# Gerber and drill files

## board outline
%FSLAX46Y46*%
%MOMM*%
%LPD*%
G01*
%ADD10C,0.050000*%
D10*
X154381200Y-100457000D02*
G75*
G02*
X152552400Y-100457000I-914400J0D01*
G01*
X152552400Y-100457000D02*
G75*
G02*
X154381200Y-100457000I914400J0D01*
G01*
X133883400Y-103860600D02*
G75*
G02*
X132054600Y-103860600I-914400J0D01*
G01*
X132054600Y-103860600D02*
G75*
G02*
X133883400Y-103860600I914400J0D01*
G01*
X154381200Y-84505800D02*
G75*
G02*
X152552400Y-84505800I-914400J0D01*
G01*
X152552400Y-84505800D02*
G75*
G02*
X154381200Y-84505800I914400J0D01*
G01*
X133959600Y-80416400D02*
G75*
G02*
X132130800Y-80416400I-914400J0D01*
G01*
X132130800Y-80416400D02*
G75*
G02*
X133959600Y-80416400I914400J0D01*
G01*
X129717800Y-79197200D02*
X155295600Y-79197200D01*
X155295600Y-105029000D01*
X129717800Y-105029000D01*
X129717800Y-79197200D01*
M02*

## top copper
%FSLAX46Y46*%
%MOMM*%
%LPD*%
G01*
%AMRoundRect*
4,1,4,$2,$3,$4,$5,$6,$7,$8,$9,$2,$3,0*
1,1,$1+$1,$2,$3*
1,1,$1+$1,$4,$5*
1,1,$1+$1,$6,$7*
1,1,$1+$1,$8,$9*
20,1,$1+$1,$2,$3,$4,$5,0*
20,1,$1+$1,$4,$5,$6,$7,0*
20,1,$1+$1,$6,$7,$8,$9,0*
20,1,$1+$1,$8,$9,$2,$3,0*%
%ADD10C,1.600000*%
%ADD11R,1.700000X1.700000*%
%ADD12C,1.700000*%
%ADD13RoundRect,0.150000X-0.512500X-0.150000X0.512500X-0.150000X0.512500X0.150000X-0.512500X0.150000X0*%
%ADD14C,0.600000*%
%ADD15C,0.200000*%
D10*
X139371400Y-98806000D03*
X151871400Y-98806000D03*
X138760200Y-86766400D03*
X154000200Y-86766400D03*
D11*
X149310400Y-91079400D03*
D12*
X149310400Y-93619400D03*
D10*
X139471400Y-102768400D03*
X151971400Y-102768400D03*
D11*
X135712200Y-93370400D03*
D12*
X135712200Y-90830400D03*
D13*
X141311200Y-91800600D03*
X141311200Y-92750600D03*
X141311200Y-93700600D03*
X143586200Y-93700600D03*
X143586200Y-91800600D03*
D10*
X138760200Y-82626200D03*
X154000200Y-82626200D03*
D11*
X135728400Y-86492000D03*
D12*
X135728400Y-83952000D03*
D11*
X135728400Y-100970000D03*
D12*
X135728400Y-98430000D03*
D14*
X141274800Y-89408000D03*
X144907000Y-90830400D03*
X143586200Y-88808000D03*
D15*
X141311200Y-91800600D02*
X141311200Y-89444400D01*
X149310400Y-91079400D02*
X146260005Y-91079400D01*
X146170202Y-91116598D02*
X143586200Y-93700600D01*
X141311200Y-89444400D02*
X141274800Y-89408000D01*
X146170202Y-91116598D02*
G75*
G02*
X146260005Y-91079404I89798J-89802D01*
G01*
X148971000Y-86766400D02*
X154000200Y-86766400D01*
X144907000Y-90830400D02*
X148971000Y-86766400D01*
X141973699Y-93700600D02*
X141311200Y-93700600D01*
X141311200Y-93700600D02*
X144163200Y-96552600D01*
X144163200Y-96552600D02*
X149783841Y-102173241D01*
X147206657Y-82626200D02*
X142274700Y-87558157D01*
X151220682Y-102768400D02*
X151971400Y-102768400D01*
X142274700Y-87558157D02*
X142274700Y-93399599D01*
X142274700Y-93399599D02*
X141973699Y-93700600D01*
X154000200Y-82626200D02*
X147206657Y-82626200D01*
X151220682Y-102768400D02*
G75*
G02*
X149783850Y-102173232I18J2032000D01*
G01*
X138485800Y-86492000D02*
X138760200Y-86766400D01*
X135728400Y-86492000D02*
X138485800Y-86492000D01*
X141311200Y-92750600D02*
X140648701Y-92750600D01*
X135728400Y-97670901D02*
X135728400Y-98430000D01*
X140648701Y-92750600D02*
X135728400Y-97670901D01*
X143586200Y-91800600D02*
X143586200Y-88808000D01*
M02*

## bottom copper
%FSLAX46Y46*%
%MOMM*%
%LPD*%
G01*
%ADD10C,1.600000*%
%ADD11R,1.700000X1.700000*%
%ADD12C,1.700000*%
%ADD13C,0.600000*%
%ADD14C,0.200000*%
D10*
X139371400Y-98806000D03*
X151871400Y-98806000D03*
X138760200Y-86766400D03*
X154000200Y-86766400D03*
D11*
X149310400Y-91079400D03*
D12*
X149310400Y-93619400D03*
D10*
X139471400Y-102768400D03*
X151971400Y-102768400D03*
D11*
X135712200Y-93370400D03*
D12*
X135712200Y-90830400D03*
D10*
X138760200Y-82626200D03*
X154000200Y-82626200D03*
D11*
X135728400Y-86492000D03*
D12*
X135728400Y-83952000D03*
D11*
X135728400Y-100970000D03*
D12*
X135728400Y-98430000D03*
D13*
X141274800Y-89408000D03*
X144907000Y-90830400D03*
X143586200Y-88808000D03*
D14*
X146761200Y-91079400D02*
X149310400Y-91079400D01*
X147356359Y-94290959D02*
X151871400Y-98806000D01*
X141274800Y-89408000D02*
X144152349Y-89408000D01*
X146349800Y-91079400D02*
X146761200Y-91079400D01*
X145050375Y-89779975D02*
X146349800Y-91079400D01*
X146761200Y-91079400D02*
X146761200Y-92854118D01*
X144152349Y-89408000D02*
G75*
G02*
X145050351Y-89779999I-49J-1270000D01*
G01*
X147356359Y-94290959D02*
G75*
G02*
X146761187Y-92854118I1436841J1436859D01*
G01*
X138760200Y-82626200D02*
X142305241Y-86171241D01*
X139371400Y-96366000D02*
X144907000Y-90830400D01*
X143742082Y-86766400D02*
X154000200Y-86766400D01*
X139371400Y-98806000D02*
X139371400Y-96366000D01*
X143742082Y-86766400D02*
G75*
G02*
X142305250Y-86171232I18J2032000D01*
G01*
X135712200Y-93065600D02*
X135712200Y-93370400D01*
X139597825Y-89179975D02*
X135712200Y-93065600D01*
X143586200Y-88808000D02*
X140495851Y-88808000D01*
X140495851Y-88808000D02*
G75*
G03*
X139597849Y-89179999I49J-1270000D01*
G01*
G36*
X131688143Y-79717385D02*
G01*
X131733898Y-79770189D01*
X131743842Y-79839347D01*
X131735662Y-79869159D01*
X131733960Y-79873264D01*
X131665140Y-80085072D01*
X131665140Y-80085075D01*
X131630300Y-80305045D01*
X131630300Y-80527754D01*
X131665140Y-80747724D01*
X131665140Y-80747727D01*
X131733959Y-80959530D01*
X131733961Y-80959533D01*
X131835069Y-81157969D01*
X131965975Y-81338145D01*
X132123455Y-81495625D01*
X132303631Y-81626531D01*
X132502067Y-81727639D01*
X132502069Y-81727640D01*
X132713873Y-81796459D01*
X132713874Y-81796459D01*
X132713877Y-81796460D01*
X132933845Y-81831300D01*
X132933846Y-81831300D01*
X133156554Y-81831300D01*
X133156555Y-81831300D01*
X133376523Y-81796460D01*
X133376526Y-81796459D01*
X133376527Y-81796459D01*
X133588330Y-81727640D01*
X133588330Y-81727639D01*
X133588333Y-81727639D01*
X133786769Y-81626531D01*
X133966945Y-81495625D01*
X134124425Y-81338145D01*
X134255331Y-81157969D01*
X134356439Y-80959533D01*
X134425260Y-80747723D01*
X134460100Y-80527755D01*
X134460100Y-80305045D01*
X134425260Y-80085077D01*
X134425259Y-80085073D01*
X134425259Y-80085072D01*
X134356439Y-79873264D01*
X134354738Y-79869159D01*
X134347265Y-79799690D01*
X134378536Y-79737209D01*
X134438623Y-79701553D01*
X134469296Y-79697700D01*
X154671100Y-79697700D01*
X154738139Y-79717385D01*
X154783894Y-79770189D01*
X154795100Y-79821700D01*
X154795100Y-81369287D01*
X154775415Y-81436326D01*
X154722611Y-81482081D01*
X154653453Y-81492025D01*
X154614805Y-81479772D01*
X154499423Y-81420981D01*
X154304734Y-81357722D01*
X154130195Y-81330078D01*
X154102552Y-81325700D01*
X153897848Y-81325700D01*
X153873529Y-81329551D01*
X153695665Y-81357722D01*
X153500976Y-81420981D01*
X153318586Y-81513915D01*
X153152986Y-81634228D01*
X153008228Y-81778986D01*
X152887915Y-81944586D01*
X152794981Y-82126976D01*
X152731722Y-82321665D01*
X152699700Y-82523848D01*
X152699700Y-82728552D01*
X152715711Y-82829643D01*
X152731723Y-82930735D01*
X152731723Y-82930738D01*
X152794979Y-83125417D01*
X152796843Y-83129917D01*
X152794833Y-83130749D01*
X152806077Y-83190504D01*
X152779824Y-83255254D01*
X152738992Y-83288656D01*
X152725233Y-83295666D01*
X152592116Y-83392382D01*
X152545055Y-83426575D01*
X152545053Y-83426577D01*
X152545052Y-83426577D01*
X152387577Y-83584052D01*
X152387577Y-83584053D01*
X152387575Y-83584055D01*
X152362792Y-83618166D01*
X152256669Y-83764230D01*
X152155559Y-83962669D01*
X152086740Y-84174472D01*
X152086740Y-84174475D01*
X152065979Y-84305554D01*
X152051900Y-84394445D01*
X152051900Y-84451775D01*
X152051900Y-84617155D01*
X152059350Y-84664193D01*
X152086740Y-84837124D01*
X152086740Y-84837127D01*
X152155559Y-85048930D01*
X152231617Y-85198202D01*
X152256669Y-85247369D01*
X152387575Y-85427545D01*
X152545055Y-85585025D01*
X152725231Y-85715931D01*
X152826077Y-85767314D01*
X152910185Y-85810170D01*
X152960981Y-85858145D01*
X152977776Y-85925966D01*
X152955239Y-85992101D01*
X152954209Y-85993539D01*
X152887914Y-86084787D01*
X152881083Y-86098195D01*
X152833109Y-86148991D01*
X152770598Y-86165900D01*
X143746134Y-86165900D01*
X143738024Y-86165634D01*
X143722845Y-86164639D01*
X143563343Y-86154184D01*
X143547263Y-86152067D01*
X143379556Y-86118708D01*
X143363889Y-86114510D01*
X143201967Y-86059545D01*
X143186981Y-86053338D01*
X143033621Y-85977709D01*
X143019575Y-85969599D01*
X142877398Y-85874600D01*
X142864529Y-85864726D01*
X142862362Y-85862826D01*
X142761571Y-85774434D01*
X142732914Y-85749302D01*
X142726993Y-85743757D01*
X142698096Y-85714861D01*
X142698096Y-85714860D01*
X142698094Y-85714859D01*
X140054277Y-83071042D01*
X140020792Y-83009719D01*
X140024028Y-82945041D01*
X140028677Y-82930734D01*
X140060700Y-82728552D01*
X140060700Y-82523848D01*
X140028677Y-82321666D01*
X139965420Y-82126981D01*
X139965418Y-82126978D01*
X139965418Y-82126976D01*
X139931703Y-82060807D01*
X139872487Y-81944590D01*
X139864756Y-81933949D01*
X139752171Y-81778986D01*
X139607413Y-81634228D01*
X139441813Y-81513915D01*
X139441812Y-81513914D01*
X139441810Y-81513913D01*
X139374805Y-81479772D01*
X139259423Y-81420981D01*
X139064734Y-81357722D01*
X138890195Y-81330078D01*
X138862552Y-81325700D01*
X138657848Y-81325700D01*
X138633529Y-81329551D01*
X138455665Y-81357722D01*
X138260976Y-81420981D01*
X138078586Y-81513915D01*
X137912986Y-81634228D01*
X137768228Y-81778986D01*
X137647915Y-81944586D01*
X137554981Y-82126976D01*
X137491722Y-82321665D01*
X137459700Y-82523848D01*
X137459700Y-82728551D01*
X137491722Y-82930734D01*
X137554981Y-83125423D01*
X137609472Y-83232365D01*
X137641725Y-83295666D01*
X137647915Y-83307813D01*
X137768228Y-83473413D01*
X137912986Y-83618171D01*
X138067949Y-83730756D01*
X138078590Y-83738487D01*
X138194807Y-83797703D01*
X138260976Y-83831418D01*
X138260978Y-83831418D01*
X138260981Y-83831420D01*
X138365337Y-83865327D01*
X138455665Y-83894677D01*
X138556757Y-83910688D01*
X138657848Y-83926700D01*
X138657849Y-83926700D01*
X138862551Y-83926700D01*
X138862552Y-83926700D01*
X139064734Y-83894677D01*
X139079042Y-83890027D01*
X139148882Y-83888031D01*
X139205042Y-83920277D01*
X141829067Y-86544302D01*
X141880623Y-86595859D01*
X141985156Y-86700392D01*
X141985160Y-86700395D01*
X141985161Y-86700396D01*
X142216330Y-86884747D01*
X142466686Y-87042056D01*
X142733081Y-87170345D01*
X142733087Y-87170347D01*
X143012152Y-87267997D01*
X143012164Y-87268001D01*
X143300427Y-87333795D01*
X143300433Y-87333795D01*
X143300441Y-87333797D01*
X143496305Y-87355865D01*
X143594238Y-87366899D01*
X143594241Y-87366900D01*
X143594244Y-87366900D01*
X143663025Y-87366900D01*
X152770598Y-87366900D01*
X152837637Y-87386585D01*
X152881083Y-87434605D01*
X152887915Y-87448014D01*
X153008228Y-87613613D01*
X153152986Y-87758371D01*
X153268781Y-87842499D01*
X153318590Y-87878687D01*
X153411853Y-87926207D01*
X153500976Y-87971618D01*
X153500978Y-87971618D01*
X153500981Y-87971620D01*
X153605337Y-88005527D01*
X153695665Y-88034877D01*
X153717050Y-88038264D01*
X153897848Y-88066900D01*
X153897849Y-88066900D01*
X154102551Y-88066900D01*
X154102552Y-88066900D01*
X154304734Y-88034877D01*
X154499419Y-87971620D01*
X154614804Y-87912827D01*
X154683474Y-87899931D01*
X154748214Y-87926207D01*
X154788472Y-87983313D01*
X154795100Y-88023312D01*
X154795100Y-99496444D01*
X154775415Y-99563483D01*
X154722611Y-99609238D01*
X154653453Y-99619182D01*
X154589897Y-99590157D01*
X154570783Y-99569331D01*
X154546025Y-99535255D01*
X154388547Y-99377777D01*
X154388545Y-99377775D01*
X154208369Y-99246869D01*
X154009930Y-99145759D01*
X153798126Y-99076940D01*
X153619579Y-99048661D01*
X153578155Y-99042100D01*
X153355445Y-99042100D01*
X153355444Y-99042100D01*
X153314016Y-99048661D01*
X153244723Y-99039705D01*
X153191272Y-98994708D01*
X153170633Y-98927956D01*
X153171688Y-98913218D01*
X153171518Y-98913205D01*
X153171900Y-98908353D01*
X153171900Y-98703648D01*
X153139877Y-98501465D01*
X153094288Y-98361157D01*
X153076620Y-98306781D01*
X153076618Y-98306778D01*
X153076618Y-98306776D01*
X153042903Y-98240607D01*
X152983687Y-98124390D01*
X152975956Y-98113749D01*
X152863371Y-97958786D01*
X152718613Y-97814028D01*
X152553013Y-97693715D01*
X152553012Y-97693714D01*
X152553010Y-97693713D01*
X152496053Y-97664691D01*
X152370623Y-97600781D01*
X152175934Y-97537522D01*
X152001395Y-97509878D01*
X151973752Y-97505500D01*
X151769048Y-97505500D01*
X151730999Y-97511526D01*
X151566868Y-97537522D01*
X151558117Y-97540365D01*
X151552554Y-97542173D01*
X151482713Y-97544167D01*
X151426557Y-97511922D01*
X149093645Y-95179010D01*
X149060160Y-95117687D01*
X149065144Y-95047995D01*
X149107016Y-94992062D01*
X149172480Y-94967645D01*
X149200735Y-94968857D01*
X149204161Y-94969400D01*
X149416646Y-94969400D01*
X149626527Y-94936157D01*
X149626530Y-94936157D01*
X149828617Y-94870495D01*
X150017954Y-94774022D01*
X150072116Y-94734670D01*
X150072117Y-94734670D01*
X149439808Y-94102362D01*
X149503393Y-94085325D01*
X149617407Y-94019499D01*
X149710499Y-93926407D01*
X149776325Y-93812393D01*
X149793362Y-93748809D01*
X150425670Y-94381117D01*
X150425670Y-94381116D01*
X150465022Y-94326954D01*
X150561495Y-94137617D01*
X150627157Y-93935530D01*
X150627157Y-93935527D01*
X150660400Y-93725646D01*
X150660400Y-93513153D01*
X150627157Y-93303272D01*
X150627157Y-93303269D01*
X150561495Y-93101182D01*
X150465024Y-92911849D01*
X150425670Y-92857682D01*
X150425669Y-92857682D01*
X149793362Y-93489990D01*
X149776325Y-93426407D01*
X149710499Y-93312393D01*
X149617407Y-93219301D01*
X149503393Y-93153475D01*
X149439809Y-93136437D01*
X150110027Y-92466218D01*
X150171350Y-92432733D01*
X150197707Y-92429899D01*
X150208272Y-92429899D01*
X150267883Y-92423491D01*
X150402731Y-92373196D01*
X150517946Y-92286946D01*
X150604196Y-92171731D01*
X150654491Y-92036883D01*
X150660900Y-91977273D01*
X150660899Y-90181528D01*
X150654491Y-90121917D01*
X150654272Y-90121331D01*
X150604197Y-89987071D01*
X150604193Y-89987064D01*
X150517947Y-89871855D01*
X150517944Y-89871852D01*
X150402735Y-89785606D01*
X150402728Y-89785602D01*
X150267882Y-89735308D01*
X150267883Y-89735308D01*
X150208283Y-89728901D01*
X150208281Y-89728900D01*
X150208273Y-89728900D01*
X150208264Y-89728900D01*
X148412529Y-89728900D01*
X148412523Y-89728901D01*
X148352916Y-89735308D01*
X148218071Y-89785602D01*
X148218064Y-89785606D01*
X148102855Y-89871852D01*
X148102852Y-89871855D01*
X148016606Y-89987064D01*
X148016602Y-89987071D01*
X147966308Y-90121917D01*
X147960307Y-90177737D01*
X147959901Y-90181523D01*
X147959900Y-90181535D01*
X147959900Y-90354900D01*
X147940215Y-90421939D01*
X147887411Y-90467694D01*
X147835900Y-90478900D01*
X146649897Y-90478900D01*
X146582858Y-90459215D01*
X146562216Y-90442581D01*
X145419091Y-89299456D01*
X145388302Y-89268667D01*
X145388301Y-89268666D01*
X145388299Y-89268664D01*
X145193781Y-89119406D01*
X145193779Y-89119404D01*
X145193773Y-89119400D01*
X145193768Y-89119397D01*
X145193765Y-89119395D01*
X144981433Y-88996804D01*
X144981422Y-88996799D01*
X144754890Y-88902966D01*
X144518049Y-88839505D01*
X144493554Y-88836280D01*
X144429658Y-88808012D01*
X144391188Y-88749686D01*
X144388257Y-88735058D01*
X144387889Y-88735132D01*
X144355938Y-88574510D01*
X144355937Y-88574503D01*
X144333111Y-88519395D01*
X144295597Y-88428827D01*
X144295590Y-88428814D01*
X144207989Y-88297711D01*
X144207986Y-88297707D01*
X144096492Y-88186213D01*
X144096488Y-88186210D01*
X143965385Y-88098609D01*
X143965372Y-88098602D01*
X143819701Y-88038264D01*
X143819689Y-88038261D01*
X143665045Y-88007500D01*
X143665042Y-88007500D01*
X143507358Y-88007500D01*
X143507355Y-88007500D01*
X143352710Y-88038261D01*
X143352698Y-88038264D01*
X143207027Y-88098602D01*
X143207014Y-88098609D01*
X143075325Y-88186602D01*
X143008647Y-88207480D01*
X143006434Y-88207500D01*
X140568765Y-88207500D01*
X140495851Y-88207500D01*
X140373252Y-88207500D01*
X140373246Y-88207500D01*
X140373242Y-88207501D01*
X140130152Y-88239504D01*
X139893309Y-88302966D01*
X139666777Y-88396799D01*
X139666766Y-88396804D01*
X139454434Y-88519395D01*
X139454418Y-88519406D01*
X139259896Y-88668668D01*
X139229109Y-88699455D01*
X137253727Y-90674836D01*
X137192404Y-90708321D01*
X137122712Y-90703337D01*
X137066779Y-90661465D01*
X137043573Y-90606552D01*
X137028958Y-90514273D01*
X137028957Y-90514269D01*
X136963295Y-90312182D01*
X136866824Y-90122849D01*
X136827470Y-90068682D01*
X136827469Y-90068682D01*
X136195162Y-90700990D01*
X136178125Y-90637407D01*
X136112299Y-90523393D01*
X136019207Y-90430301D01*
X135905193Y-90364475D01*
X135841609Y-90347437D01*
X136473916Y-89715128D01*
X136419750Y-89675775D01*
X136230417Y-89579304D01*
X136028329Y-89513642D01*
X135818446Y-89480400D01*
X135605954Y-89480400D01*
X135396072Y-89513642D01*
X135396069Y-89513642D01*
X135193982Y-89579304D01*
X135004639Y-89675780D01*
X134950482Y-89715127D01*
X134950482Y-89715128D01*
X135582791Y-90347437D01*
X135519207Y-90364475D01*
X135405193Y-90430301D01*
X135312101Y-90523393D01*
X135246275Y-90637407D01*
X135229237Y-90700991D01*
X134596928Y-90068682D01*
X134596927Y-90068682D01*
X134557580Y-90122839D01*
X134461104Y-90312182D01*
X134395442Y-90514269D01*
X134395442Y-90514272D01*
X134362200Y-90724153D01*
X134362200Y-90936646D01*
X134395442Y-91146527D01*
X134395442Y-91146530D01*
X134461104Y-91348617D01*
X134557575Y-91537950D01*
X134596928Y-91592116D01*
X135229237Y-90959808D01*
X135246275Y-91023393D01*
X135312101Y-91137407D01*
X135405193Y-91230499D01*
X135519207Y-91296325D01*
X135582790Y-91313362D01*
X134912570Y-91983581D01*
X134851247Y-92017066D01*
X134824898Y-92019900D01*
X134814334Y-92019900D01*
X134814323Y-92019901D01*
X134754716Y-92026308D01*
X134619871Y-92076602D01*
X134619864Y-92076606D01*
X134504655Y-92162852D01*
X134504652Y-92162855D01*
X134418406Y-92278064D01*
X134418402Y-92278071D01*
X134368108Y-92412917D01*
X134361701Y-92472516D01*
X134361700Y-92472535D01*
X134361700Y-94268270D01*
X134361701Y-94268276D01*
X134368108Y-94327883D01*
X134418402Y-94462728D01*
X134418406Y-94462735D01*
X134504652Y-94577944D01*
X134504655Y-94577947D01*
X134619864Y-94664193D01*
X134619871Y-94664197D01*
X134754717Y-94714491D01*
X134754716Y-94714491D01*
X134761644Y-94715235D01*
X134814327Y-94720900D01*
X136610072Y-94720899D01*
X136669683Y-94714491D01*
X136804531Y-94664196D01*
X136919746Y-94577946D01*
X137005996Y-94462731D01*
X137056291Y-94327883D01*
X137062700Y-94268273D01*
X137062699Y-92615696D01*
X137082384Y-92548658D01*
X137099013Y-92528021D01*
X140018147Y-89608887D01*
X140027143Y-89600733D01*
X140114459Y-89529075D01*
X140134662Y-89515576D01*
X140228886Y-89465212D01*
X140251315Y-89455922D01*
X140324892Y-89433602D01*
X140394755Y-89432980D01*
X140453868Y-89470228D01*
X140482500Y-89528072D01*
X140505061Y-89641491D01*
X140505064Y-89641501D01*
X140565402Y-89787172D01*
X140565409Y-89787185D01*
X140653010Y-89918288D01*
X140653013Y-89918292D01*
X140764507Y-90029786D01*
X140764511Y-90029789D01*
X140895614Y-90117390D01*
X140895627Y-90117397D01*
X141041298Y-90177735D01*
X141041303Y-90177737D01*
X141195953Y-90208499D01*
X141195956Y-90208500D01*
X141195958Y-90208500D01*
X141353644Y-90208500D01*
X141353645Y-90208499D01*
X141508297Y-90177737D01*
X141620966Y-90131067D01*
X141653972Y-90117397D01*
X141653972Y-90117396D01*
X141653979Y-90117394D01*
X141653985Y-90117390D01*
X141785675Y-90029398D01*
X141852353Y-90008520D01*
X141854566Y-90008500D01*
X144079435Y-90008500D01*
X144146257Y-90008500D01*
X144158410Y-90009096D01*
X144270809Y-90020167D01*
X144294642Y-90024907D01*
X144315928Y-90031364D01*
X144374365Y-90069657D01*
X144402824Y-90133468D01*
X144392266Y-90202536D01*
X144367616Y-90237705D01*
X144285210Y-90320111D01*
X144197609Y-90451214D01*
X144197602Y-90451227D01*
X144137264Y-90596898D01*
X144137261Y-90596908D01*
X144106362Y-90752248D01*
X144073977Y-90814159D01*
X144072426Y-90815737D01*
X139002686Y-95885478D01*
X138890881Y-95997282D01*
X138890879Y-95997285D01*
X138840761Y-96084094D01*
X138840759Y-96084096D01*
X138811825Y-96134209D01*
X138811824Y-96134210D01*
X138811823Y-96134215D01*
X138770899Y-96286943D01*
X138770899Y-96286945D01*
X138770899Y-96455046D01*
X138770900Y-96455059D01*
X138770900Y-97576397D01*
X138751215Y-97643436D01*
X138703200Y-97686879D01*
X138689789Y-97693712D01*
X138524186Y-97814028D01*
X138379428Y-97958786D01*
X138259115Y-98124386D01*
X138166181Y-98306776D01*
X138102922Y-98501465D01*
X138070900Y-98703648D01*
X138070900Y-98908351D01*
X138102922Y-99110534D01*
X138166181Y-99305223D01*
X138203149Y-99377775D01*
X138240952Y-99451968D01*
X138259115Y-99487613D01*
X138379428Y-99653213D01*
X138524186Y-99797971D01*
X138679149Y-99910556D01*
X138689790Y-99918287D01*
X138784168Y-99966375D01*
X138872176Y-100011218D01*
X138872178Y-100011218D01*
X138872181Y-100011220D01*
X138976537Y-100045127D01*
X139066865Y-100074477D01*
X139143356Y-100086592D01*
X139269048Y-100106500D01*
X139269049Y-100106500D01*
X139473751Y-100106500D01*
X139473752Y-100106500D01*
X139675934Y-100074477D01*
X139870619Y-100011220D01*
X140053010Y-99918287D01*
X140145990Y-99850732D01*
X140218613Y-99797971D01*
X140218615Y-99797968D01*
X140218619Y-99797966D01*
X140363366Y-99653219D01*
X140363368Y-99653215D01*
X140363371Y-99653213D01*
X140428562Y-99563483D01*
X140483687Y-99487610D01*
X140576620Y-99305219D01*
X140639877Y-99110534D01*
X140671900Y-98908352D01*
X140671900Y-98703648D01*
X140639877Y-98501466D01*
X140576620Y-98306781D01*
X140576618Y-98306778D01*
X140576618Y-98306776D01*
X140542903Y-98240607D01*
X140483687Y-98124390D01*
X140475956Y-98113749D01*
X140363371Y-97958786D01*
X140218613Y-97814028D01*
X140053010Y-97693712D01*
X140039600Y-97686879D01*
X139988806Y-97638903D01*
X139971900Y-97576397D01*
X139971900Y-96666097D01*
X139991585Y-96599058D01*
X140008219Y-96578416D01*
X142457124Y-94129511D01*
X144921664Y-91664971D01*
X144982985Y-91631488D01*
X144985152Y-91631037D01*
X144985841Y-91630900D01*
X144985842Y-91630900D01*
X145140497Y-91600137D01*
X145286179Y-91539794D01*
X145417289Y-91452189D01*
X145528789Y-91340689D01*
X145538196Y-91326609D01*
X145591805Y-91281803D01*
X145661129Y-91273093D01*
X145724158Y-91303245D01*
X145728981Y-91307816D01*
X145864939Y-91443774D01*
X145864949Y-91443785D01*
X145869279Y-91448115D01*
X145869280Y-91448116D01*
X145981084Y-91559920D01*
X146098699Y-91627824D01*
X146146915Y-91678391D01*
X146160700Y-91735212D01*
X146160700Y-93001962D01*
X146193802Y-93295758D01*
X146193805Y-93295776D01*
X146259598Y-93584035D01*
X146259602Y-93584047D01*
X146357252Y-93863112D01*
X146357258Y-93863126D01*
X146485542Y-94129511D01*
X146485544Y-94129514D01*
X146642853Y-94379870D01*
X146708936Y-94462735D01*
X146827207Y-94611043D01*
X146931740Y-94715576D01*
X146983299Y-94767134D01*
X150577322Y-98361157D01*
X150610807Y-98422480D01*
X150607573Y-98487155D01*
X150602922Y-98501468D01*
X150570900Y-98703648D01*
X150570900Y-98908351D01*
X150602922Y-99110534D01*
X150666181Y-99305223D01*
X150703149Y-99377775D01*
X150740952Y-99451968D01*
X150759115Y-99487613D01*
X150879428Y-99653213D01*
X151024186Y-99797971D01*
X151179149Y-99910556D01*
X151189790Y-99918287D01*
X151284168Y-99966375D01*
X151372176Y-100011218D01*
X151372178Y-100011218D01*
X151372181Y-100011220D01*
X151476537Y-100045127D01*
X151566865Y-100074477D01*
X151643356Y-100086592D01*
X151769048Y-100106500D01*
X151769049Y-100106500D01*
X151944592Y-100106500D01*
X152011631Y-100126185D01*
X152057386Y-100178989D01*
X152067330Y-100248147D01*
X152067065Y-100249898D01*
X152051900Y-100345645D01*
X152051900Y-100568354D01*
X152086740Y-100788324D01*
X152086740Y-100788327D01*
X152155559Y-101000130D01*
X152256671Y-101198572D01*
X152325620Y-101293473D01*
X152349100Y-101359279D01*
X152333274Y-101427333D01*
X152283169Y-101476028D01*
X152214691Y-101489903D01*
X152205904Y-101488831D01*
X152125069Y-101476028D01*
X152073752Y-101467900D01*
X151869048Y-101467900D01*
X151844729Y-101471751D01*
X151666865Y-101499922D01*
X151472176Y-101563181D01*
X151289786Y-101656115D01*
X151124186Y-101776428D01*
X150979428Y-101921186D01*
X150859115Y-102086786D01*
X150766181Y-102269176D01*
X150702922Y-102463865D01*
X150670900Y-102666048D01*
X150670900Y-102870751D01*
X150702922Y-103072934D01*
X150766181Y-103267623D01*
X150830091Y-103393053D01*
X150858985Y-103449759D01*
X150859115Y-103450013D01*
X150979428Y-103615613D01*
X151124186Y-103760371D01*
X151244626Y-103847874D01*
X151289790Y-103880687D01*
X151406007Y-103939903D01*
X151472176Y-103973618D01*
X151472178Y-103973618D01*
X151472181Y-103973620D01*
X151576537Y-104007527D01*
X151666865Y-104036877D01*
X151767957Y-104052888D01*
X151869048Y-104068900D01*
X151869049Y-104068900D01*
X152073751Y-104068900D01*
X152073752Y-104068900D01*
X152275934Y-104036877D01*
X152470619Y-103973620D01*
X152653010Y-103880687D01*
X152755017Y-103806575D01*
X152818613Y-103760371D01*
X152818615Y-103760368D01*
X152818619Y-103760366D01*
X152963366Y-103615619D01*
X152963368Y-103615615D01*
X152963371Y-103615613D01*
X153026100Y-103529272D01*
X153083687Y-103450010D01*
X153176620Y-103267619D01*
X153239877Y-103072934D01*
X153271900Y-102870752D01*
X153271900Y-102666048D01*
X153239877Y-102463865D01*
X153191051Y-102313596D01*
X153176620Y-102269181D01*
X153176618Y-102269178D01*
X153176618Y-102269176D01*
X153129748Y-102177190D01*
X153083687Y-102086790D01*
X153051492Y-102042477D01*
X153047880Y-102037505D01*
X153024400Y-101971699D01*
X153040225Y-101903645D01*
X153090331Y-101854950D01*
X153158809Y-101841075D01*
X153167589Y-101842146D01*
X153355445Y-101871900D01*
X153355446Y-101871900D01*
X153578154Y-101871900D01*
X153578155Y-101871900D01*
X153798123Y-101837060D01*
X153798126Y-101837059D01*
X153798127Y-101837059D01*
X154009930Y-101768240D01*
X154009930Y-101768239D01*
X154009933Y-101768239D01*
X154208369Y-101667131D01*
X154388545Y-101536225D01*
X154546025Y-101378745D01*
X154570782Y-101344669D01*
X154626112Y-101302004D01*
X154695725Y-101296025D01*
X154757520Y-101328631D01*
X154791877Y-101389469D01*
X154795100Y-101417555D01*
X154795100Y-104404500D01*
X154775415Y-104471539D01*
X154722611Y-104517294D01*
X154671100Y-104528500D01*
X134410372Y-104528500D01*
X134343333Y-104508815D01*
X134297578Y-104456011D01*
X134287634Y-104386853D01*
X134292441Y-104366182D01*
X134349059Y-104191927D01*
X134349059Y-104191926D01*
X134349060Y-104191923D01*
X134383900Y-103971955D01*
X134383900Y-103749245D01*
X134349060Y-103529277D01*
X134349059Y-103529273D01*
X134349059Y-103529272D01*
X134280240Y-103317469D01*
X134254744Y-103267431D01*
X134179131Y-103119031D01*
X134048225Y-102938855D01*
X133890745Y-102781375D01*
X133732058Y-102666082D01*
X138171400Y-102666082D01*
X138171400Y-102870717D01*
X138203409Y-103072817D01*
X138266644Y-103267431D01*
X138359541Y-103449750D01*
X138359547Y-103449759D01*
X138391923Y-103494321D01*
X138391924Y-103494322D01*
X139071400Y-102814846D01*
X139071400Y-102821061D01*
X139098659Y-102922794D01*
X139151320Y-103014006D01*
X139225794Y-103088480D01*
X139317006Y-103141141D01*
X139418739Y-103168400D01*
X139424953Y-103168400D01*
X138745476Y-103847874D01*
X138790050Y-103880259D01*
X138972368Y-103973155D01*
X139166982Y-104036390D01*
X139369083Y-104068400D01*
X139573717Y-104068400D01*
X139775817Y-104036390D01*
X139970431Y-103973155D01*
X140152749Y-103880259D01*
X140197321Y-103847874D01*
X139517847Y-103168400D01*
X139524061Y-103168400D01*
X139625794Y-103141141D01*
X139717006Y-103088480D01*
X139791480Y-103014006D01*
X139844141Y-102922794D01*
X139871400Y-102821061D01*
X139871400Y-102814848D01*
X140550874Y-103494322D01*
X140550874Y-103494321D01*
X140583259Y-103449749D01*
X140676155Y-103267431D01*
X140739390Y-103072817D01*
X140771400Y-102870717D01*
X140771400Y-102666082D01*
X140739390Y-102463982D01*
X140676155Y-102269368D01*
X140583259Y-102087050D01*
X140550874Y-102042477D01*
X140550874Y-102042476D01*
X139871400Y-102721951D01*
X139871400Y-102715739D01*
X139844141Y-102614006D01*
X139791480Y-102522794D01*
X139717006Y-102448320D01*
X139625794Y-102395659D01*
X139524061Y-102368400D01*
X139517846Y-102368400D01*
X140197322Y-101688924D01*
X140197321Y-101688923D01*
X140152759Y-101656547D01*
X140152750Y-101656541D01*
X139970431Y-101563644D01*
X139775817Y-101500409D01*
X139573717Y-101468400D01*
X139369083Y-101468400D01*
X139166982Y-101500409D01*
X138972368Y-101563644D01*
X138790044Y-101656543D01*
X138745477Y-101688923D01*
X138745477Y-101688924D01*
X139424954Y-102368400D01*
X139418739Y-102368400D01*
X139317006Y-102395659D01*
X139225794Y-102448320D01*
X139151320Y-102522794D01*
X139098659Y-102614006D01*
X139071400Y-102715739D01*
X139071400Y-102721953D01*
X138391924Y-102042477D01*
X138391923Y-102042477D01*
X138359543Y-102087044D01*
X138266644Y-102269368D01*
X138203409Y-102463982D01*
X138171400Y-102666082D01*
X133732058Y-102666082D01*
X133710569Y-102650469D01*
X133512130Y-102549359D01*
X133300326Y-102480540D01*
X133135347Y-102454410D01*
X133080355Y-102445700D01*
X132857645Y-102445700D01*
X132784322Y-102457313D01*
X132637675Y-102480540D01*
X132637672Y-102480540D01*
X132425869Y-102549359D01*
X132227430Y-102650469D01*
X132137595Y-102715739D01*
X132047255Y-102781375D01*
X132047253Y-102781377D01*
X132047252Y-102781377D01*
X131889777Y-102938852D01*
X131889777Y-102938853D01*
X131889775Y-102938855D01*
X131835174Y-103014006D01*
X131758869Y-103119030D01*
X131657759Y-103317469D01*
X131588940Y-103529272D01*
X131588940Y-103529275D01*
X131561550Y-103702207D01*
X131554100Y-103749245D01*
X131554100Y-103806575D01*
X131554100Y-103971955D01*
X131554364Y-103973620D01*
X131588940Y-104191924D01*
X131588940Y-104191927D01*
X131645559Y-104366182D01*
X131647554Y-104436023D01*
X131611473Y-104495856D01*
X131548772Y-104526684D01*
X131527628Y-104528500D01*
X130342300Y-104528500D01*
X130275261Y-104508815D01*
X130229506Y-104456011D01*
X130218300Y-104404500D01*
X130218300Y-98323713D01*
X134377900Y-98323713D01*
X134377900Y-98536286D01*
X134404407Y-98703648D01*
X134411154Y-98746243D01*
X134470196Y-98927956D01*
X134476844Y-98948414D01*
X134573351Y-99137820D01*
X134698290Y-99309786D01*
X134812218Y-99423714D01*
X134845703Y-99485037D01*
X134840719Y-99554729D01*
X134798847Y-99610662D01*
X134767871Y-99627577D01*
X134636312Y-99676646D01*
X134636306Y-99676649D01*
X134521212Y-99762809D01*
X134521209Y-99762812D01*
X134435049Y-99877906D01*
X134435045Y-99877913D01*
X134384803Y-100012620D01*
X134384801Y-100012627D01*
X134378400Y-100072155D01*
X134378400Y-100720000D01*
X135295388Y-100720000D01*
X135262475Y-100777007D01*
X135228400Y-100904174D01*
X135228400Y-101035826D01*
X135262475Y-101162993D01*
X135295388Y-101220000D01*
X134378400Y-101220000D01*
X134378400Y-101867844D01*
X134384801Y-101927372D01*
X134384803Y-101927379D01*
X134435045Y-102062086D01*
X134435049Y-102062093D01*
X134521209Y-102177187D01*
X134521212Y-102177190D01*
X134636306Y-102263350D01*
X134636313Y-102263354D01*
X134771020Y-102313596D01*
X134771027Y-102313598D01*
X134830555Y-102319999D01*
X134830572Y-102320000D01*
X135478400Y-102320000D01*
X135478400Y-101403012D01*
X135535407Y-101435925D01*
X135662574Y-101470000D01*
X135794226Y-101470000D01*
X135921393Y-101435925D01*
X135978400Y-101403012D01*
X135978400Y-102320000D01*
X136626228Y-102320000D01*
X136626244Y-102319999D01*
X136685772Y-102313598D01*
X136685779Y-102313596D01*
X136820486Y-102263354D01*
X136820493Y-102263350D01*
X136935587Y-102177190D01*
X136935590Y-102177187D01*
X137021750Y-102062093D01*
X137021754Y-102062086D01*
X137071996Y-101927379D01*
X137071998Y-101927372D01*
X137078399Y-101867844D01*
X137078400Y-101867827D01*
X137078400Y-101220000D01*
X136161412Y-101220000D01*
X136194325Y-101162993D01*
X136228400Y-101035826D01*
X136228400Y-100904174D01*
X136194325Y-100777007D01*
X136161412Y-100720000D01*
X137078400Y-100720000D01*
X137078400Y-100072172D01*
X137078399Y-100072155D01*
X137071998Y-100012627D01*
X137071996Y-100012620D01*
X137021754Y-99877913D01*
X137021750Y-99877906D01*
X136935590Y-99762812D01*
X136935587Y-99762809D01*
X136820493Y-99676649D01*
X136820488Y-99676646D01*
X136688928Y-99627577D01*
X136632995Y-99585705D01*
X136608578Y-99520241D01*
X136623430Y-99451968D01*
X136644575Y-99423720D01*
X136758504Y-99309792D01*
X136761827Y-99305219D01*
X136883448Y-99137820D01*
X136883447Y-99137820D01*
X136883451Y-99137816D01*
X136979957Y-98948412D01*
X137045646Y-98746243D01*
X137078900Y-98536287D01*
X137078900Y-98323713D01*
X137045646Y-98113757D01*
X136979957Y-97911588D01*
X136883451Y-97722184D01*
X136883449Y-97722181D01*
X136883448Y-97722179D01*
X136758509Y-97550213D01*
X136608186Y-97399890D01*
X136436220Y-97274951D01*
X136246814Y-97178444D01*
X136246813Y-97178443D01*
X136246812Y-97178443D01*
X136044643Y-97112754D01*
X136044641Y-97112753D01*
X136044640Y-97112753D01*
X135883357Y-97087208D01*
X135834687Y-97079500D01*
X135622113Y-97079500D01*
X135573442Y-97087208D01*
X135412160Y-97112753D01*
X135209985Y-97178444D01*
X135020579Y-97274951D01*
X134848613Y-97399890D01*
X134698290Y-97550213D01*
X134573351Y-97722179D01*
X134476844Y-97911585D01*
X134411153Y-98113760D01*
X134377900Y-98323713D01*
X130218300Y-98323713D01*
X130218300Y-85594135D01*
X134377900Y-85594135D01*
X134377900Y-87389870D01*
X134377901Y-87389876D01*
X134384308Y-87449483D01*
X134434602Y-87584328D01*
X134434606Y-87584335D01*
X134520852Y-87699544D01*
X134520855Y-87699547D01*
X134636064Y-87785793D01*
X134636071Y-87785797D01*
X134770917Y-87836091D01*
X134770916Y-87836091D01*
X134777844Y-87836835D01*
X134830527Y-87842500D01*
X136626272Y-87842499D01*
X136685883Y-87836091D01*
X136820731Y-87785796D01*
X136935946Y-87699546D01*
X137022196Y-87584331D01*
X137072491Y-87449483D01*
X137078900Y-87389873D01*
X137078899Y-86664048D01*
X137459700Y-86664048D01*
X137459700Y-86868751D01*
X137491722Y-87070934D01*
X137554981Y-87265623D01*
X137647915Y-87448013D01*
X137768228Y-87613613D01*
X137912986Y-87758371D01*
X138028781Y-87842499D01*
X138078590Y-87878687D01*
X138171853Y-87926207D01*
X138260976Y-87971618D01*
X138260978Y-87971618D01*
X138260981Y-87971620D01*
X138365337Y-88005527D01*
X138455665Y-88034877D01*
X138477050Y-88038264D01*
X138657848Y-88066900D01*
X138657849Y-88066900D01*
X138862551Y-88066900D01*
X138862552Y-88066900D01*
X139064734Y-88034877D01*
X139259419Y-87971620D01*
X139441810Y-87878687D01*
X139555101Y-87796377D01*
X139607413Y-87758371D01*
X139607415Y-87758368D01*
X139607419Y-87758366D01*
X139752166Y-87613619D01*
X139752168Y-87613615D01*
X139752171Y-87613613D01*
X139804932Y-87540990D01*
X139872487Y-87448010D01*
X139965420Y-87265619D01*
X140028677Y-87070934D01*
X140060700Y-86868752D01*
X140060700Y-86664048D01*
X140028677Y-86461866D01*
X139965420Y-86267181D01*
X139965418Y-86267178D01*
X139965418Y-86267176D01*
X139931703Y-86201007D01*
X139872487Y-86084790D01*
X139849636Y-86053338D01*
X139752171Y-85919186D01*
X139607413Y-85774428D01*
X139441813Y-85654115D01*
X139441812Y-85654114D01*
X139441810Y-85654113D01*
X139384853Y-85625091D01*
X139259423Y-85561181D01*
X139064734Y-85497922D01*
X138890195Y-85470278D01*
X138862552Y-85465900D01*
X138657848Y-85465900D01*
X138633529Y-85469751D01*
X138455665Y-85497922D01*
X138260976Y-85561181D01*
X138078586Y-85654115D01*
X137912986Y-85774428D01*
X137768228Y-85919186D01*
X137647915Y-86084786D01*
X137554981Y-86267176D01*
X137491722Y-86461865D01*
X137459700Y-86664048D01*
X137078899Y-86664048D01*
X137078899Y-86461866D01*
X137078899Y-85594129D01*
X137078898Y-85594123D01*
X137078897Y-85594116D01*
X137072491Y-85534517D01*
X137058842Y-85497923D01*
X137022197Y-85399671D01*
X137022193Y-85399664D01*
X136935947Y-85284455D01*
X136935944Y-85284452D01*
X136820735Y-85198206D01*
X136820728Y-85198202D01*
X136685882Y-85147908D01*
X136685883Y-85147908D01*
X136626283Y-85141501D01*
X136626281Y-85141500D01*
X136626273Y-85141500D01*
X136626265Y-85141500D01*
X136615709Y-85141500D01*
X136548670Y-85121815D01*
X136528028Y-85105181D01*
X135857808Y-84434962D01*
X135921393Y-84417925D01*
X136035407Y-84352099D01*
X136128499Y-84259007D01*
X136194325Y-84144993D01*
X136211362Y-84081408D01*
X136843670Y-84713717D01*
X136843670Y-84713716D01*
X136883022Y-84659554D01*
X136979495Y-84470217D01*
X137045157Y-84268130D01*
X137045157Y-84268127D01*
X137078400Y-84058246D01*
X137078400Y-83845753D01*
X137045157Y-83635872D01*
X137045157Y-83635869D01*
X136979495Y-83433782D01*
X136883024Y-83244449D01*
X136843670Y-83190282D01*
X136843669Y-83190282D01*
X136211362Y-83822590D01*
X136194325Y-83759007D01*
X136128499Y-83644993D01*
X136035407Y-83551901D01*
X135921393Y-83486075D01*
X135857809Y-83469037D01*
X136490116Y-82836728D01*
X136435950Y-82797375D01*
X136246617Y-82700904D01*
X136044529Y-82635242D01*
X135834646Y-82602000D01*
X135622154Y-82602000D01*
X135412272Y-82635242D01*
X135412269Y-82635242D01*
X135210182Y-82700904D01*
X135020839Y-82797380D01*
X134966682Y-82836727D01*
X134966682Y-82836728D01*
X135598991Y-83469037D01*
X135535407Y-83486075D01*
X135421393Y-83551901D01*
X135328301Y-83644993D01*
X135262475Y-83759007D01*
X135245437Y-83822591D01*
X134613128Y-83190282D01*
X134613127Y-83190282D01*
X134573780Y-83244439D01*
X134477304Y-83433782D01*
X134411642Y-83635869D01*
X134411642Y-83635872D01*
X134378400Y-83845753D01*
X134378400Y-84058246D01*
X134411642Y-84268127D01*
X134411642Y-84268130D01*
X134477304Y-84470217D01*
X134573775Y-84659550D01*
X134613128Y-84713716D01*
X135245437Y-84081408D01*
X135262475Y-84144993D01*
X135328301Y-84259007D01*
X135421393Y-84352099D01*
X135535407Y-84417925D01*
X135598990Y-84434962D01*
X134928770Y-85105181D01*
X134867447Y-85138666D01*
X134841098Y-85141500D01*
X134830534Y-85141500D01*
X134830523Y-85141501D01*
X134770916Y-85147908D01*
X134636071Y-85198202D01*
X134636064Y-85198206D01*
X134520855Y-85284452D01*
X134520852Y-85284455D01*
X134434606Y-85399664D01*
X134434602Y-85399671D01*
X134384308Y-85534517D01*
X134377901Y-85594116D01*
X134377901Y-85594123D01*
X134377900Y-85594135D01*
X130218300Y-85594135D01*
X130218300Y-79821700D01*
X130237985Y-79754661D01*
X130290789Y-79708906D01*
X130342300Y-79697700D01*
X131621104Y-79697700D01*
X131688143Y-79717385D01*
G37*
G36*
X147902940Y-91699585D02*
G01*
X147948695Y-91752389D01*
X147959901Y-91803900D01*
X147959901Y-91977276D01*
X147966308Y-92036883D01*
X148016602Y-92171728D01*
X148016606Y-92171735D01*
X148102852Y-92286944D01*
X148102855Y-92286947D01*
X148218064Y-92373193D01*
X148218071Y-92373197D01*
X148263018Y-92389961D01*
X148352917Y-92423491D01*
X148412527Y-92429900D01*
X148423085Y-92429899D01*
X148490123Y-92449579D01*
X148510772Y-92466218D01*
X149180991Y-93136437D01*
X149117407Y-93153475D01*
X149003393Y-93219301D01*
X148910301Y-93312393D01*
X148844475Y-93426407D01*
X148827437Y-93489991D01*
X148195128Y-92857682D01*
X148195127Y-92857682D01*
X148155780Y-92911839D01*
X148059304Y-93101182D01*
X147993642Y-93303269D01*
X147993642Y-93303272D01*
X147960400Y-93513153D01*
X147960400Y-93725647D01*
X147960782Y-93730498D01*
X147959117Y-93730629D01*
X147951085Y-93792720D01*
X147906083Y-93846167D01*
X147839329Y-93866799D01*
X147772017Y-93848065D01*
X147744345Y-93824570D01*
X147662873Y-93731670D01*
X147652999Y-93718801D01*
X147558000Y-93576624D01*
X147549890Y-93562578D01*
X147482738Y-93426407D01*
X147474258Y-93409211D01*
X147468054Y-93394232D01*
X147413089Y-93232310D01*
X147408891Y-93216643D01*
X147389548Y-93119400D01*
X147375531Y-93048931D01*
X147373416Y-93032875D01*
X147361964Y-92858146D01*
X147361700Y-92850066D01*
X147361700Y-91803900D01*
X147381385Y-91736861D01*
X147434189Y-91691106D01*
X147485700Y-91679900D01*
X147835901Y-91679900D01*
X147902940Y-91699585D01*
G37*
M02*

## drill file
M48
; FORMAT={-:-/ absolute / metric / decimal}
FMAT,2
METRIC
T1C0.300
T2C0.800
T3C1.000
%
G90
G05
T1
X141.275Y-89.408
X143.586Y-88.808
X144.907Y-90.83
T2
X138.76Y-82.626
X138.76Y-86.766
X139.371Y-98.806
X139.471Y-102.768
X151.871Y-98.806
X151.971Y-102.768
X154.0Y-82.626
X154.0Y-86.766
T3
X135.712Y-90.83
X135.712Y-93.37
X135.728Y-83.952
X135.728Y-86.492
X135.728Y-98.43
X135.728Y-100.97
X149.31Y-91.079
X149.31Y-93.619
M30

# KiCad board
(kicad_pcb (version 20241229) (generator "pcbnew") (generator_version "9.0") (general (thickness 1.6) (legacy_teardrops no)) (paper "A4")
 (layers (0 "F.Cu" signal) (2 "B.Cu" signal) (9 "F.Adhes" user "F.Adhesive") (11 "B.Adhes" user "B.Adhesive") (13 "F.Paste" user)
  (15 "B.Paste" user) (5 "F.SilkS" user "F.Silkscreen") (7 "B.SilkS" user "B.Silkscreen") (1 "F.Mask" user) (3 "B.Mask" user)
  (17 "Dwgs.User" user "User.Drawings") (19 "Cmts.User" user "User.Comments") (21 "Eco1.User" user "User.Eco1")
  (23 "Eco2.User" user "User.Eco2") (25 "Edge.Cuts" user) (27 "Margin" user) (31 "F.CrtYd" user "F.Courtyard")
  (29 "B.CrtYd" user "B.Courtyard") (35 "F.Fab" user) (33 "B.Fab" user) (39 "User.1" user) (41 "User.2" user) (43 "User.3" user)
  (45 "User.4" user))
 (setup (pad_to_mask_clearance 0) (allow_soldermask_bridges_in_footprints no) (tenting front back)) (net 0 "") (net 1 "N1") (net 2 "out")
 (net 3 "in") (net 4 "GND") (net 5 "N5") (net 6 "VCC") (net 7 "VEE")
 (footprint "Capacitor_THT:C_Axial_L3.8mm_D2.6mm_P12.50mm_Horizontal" (layer "F.Cu") (at 139.3714 98.806)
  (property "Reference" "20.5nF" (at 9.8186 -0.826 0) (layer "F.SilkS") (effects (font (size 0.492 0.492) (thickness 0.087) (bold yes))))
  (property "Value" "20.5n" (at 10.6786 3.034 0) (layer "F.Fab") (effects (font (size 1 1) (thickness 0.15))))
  (pad "1" thru_hole circle (at 0 0) (size 1.6 1.6) (drill 0.8) (layers "*.Cu" "*.Mask") (remove_unused_layers no) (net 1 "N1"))
  (pad "2" thru_hole circle (at 12.5 0) (size 1.6 1.6) (drill 0.8) (layers "*.Cu" "*.Mask") (remove_unused_layers no) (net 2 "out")))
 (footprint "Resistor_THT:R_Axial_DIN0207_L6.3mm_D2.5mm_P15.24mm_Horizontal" (layer "F.Cu") (at 138.7602 86.7664)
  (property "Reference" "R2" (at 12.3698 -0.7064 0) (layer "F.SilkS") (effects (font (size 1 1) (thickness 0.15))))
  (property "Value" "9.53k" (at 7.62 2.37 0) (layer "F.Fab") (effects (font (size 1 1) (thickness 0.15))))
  (pad "1" thru_hole circle (at 0 0) (size 1.6 1.6) (drill 0.8) (layers "*.Cu" "*.Mask") (remove_unused_layers no) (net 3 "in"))
  (pad "2" thru_hole circle (at 15.24 0) (size 1.6 1.6) (drill 0.8) (layers "*.Cu" "*.Mask") (remove_unused_layers no) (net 1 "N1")))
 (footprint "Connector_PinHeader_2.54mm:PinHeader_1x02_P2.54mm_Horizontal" (layer "F.Cu") (at 149.3104 91.0794)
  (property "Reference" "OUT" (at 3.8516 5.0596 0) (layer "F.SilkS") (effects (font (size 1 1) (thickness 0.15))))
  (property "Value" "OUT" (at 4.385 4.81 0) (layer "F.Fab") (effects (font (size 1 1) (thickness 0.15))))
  (pad "1" thru_hole rect (at 0 0) (size 1.7 1.7) (drill 1) (layers "*.Cu" "*.Mask") (remove_unused_layers no) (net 2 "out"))
  (pad "2" thru_hole circle (at 0 2.54) (size 1.7 1.7) (drill 1) (layers "*.Cu" "*.Mask") (remove_unused_layers no) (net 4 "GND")))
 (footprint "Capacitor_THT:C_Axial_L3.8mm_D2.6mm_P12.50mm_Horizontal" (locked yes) (layer "F.Cu") (at 139.4714 102.7684)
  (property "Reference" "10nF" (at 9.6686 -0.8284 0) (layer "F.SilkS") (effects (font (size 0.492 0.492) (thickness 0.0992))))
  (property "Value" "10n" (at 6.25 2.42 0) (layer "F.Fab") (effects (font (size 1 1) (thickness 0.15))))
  (pad "1" thru_hole circle (at 0 0) (size 1.6 1.6) (drill 0.8) (layers "*.Cu" "*.Mask") (remove_unused_layers no) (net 4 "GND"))
  (pad "2" thru_hole circle (at 12.5 0) (size 1.6 1.6) (drill 0.8) (layers "*.Cu" "*.Mask") (remove_unused_layers no) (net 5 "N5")))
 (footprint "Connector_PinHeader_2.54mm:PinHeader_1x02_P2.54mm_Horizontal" (layer "F.Cu") (at 135.7122 93.3704 180)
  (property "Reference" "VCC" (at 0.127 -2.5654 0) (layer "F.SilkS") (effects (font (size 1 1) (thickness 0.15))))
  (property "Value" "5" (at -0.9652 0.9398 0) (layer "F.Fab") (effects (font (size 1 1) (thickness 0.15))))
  (pad "1" thru_hole rect (at 0 0 180) (size 1.7 1.7) (drill 1) (layers "*.Cu" "*.Mask") (remove_unused_layers no) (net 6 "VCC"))
  (pad "2" thru_hole circle (at 0 2.54 180) (size 1.7 1.7) (drill 1) (layers "*.Cu" "*.Mask") (remove_unused_layers no) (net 4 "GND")))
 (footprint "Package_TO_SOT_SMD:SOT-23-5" (layer "F.Cu") (at 142.4487 92.7506)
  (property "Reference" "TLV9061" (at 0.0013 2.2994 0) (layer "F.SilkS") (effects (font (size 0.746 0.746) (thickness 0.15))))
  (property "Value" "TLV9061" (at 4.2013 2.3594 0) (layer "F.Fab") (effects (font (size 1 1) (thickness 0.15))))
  (pad "1" smd roundrect (at -1.1375 -0.95) (size 1.325 0.6) (layers "F.Cu" "F.Mask" "F.Paste") (roundrect_rratio 0.25) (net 2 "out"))
  (pad "2" smd roundrect (at -1.1375 0) (size 1.325 0.6) (layers "F.Cu" "F.Mask" "F.Paste") (roundrect_rratio 0.25) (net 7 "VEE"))
  (pad "3" smd roundrect (at -1.1375 0.95) (size 1.325 0.6) (layers "F.Cu" "F.Mask" "F.Paste") (roundrect_rratio 0.25) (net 5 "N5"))
  (pad "4" smd roundrect (at 1.1375 0.95) (size 1.325 0.6) (layers "F.Cu" "F.Mask" "F.Paste") (roundrect_rratio 0.25) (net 2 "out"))
  (pad "5" smd roundrect (at 1.1375 -0.95) (size 1.325 0.6) (layers "F.Cu" "F.Mask" "F.Paste") (roundrect_rratio 0.25) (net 6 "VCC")))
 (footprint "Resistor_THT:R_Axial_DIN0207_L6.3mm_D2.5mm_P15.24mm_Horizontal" (layer "F.Cu") (at 138.7602 82.6262)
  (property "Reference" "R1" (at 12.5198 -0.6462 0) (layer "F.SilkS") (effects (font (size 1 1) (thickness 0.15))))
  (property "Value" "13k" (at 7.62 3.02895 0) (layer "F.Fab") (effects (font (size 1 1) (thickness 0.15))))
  (pad "1" thru_hole circle (at 0 0) (size 1.6 1.6) (drill 0.8) (layers "*.Cu" "*.Mask") (remove_unused_layers no) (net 1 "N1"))
  (pad "2" thru_hole circle (at 15.24 0) (size 1.6 1.6) (drill 0.8) (layers "*.Cu" "*.Mask") (remove_unused_layers no) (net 5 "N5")))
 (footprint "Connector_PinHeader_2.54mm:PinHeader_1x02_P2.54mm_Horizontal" (layer "F.Cu") (at 135.7284 86.492 180)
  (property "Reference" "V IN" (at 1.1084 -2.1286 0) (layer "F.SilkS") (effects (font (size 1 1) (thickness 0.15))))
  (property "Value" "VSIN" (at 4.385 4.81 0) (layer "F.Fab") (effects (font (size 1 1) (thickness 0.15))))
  (pad "1" thru_hole rect (at 0 0 180) (size 1.7 1.7) (drill 1) (layers "*.Cu" "*.Mask") (remove_unused_layers no) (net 3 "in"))
  (pad "2" thru_hole circle (at 0 2.54 180) (size 1.7 1.7) (drill 1) (layers "*.Cu" "*.Mask") (remove_unused_layers no) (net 4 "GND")))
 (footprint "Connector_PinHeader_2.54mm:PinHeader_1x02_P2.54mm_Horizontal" (layer "F.Cu") (at 135.7284 100.97 180)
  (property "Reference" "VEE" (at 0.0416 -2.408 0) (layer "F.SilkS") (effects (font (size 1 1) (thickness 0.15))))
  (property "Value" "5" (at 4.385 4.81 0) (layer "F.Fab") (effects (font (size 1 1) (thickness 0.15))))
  (pad "1" thru_hole rect (at 0 0 180) (size 1.7 1.7) (drill 1) (layers "*.Cu" "*.Mask") (remove_unused_layers no) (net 4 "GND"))
  (pad "2" thru_hole circle (at 0 2.54 180) (size 1.7 1.7) (drill 1) (layers "*.Cu" "*.Mask") (remove_unused_layers no) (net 7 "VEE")))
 (gr_circle (center 153.4668 100.457) (end 154.3812 100.457) (stroke (width 0.05) (type default)) (fill no) (layer "Edge.Cuts"))
 (gr_circle (center 132.969 103.8606) (end 133.8834 103.8606) (stroke (width 0.05) (type default)) (fill no) (layer "Edge.Cuts"))
 (gr_circle (center 153.4668 84.5058) (end 154.3812 84.5058) (stroke (width 0.05) (type default)) (fill no) (layer "Edge.Cuts"))
 (gr_circle (center 133.0452 80.4164) (end 133.9596 80.4164) (stroke (width 0.05) (type default)) (fill no) (layer "Edge.Cuts"))
 (gr_rect (start 129.7178 79.1972) (end 155.2956 105.029) (stroke (width 0.05) (type default)) (fill no) (layer "Edge.Cuts"))
 (segment (start 141.3112 91.8006) (end 141.3112 89.4444) (width 0.2) (layer "F.Cu") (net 2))
 (segment (start 149.3104 91.0794) (end 146.260005 91.0794) (width 0.2) (layer "F.Cu") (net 2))
 (segment (start 146.170202 91.116598) (end 143.5862 93.7006) (width 0.2) (layer "F.Cu") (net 2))
 (segment (start 141.3112 89.4444) (end 141.2748 89.408) (width 0.2) (layer "F.Cu") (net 2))
 (via (at 141.2748 89.408) (size 0.6) (drill 0.3) (layers "F.Cu" "B.Cu") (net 2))
 (arc (start 146.170202 91.116598) (mid 146.211404 91.089068) (end 146.260005 91.0794) (width 0.2) (layer "F.Cu") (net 2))
 (segment (start 146.7612 91.0794) (end 149.3104 91.0794) (width 0.2) (layer "B.Cu") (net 2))
 (segment (start 147.356359 94.290959) (end 151.8714 98.806) (width 0.2) (layer "B.Cu") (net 2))
 (segment (start 141.2748 89.408) (end 144.152349 89.408) (width 0.2) (layer "B.Cu") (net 2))
 (segment (start 146.3498 91.0794) (end 146.7612 91.0794) (width 0.2) (layer "B.Cu") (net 2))
 (segment (start 145.050375 89.779975) (end 146.3498 91.0794) (width 0.2) (layer "B.Cu") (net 2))
 (segment (start 146.7612 91.0794) (end 146.7612 92.854118) (width 0.2) (layer "B.Cu") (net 2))
 (arc (start 144.152349 89.408) (mid 144.638357 89.504673) (end 145.050375 89.779975) (width 0.2) (layer "B.Cu") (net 2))
 (arc (start 147.356359 94.290959) (mid 146.915877 93.631731) (end 146.7612 92.854118) (width 0.2) (layer "B.Cu") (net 2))
 (segment (start 148.971 86.7664) (end 154.0002 86.7664) (width 0.2) (layer "F.Cu") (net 1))
 (segment (start 144.907 90.8304) (end 148.971 86.7664) (width 0.2) (layer "F.Cu") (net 1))
 (via (at 144.907 90.8304) (size 0.6) (drill 0.3) (layers "F.Cu" "B.Cu") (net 1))
 (segment (start 138.7602 82.6262) (end 142.305241 86.171241) (width 0.2) (layer "B.Cu") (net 1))
 (segment (start 139.3714 96.366) (end 144.907 90.8304) (width 0.2) (layer "B.Cu") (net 1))
 (segment (start 143.742082 86.7664) (end 154.0002 86.7664) (width 0.2) (layer "B.Cu") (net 1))
 (segment (start 139.3714 98.806) (end 139.3714 96.366) (width 0.2) (layer "B.Cu") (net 1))
 (arc (start 143.742082 86.7664) (mid 142.964469 86.611723) (end 142.305241 86.171241) (width 0.2) (layer "B.Cu") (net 1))
 (segment (start 141.973699 93.7006) (end 141.3112 93.7006) (width 0.2) (layer "F.Cu") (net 5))
 (segment (start 141.3112 93.7006) (end 144.1632 96.5526) (width 0.2) (layer "F.Cu") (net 5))
 (segment (start 144.1632 96.5526) (end 149.783841 102.173241) (width 0.2) (layer "F.Cu") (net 5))
 (segment (start 147.206657 82.6262) (end 142.2747 87.558157) (width 0.2) (layer "F.Cu") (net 5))
 (segment (start 151.220682 102.7684) (end 151.9714 102.7684) (width 0.2) (layer "F.Cu") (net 5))
 (segment (start 142.2747 87.558157) (end 142.2747 93.399599) (width 0.2) (layer "F.Cu") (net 5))
 (segment (start 142.2747 93.399599) (end 141.973699 93.7006) (width 0.2) (layer "F.Cu") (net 5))
 (segment (start 154.0002 82.6262) (end 147.206657 82.6262) (width 0.2) (layer "F.Cu") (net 5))
 (arc (start 151.220682 102.7684) (mid 150.443069 102.613723) (end 149.783841 102.173241) (width 0.2) (layer "F.Cu") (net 5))
 (segment (start 138.4858 86.492) (end 138.7602 86.7664) (width 0.2) (layer "F.Cu") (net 3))
 (segment (start 135.7284 86.492) (end 138.4858 86.492) (width 0.2) (layer "F.Cu") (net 3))
 (segment (start 141.3112 92.7506) (end 140.648701 92.7506) (width 0.2) (layer "F.Cu") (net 7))
 (segment (start 135.7284 97.670901) (end 135.7284 98.43) (width 0.2) (layer "F.Cu") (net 7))
 (segment (start 140.648701 92.7506) (end 135.7284 97.670901) (width 0.2) (layer "F.Cu") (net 7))
 (segment (start 143.5862 91.8006) (end 143.5862 88.808) (width 0.2) (layer "F.Cu") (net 6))
 (via (at 143.5862 88.808) (size 0.6) (drill 0.3) (layers "F.Cu" "B.Cu") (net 6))
 (segment (start 135.7122 93.0656) (end 135.7122 93.3704) (width 0.2) (layer "B.Cu") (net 6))
 (segment (start 139.597825 89.179975) (end 135.7122 93.0656) (width 0.2) (layer "B.Cu") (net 6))
 (segment (start 143.5862 88.808) (end 140.495851 88.808) (width 0.2) (layer "B.Cu") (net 6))
 (arc (start 140.495851 88.808) (mid 140.009843 88.904673) (end 139.597825 89.179975) (width 0.2) (layer "B.Cu") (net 6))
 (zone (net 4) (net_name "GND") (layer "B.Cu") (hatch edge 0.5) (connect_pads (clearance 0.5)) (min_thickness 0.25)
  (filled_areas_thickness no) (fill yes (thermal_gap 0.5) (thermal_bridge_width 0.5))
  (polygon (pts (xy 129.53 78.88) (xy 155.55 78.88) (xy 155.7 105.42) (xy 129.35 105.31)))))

